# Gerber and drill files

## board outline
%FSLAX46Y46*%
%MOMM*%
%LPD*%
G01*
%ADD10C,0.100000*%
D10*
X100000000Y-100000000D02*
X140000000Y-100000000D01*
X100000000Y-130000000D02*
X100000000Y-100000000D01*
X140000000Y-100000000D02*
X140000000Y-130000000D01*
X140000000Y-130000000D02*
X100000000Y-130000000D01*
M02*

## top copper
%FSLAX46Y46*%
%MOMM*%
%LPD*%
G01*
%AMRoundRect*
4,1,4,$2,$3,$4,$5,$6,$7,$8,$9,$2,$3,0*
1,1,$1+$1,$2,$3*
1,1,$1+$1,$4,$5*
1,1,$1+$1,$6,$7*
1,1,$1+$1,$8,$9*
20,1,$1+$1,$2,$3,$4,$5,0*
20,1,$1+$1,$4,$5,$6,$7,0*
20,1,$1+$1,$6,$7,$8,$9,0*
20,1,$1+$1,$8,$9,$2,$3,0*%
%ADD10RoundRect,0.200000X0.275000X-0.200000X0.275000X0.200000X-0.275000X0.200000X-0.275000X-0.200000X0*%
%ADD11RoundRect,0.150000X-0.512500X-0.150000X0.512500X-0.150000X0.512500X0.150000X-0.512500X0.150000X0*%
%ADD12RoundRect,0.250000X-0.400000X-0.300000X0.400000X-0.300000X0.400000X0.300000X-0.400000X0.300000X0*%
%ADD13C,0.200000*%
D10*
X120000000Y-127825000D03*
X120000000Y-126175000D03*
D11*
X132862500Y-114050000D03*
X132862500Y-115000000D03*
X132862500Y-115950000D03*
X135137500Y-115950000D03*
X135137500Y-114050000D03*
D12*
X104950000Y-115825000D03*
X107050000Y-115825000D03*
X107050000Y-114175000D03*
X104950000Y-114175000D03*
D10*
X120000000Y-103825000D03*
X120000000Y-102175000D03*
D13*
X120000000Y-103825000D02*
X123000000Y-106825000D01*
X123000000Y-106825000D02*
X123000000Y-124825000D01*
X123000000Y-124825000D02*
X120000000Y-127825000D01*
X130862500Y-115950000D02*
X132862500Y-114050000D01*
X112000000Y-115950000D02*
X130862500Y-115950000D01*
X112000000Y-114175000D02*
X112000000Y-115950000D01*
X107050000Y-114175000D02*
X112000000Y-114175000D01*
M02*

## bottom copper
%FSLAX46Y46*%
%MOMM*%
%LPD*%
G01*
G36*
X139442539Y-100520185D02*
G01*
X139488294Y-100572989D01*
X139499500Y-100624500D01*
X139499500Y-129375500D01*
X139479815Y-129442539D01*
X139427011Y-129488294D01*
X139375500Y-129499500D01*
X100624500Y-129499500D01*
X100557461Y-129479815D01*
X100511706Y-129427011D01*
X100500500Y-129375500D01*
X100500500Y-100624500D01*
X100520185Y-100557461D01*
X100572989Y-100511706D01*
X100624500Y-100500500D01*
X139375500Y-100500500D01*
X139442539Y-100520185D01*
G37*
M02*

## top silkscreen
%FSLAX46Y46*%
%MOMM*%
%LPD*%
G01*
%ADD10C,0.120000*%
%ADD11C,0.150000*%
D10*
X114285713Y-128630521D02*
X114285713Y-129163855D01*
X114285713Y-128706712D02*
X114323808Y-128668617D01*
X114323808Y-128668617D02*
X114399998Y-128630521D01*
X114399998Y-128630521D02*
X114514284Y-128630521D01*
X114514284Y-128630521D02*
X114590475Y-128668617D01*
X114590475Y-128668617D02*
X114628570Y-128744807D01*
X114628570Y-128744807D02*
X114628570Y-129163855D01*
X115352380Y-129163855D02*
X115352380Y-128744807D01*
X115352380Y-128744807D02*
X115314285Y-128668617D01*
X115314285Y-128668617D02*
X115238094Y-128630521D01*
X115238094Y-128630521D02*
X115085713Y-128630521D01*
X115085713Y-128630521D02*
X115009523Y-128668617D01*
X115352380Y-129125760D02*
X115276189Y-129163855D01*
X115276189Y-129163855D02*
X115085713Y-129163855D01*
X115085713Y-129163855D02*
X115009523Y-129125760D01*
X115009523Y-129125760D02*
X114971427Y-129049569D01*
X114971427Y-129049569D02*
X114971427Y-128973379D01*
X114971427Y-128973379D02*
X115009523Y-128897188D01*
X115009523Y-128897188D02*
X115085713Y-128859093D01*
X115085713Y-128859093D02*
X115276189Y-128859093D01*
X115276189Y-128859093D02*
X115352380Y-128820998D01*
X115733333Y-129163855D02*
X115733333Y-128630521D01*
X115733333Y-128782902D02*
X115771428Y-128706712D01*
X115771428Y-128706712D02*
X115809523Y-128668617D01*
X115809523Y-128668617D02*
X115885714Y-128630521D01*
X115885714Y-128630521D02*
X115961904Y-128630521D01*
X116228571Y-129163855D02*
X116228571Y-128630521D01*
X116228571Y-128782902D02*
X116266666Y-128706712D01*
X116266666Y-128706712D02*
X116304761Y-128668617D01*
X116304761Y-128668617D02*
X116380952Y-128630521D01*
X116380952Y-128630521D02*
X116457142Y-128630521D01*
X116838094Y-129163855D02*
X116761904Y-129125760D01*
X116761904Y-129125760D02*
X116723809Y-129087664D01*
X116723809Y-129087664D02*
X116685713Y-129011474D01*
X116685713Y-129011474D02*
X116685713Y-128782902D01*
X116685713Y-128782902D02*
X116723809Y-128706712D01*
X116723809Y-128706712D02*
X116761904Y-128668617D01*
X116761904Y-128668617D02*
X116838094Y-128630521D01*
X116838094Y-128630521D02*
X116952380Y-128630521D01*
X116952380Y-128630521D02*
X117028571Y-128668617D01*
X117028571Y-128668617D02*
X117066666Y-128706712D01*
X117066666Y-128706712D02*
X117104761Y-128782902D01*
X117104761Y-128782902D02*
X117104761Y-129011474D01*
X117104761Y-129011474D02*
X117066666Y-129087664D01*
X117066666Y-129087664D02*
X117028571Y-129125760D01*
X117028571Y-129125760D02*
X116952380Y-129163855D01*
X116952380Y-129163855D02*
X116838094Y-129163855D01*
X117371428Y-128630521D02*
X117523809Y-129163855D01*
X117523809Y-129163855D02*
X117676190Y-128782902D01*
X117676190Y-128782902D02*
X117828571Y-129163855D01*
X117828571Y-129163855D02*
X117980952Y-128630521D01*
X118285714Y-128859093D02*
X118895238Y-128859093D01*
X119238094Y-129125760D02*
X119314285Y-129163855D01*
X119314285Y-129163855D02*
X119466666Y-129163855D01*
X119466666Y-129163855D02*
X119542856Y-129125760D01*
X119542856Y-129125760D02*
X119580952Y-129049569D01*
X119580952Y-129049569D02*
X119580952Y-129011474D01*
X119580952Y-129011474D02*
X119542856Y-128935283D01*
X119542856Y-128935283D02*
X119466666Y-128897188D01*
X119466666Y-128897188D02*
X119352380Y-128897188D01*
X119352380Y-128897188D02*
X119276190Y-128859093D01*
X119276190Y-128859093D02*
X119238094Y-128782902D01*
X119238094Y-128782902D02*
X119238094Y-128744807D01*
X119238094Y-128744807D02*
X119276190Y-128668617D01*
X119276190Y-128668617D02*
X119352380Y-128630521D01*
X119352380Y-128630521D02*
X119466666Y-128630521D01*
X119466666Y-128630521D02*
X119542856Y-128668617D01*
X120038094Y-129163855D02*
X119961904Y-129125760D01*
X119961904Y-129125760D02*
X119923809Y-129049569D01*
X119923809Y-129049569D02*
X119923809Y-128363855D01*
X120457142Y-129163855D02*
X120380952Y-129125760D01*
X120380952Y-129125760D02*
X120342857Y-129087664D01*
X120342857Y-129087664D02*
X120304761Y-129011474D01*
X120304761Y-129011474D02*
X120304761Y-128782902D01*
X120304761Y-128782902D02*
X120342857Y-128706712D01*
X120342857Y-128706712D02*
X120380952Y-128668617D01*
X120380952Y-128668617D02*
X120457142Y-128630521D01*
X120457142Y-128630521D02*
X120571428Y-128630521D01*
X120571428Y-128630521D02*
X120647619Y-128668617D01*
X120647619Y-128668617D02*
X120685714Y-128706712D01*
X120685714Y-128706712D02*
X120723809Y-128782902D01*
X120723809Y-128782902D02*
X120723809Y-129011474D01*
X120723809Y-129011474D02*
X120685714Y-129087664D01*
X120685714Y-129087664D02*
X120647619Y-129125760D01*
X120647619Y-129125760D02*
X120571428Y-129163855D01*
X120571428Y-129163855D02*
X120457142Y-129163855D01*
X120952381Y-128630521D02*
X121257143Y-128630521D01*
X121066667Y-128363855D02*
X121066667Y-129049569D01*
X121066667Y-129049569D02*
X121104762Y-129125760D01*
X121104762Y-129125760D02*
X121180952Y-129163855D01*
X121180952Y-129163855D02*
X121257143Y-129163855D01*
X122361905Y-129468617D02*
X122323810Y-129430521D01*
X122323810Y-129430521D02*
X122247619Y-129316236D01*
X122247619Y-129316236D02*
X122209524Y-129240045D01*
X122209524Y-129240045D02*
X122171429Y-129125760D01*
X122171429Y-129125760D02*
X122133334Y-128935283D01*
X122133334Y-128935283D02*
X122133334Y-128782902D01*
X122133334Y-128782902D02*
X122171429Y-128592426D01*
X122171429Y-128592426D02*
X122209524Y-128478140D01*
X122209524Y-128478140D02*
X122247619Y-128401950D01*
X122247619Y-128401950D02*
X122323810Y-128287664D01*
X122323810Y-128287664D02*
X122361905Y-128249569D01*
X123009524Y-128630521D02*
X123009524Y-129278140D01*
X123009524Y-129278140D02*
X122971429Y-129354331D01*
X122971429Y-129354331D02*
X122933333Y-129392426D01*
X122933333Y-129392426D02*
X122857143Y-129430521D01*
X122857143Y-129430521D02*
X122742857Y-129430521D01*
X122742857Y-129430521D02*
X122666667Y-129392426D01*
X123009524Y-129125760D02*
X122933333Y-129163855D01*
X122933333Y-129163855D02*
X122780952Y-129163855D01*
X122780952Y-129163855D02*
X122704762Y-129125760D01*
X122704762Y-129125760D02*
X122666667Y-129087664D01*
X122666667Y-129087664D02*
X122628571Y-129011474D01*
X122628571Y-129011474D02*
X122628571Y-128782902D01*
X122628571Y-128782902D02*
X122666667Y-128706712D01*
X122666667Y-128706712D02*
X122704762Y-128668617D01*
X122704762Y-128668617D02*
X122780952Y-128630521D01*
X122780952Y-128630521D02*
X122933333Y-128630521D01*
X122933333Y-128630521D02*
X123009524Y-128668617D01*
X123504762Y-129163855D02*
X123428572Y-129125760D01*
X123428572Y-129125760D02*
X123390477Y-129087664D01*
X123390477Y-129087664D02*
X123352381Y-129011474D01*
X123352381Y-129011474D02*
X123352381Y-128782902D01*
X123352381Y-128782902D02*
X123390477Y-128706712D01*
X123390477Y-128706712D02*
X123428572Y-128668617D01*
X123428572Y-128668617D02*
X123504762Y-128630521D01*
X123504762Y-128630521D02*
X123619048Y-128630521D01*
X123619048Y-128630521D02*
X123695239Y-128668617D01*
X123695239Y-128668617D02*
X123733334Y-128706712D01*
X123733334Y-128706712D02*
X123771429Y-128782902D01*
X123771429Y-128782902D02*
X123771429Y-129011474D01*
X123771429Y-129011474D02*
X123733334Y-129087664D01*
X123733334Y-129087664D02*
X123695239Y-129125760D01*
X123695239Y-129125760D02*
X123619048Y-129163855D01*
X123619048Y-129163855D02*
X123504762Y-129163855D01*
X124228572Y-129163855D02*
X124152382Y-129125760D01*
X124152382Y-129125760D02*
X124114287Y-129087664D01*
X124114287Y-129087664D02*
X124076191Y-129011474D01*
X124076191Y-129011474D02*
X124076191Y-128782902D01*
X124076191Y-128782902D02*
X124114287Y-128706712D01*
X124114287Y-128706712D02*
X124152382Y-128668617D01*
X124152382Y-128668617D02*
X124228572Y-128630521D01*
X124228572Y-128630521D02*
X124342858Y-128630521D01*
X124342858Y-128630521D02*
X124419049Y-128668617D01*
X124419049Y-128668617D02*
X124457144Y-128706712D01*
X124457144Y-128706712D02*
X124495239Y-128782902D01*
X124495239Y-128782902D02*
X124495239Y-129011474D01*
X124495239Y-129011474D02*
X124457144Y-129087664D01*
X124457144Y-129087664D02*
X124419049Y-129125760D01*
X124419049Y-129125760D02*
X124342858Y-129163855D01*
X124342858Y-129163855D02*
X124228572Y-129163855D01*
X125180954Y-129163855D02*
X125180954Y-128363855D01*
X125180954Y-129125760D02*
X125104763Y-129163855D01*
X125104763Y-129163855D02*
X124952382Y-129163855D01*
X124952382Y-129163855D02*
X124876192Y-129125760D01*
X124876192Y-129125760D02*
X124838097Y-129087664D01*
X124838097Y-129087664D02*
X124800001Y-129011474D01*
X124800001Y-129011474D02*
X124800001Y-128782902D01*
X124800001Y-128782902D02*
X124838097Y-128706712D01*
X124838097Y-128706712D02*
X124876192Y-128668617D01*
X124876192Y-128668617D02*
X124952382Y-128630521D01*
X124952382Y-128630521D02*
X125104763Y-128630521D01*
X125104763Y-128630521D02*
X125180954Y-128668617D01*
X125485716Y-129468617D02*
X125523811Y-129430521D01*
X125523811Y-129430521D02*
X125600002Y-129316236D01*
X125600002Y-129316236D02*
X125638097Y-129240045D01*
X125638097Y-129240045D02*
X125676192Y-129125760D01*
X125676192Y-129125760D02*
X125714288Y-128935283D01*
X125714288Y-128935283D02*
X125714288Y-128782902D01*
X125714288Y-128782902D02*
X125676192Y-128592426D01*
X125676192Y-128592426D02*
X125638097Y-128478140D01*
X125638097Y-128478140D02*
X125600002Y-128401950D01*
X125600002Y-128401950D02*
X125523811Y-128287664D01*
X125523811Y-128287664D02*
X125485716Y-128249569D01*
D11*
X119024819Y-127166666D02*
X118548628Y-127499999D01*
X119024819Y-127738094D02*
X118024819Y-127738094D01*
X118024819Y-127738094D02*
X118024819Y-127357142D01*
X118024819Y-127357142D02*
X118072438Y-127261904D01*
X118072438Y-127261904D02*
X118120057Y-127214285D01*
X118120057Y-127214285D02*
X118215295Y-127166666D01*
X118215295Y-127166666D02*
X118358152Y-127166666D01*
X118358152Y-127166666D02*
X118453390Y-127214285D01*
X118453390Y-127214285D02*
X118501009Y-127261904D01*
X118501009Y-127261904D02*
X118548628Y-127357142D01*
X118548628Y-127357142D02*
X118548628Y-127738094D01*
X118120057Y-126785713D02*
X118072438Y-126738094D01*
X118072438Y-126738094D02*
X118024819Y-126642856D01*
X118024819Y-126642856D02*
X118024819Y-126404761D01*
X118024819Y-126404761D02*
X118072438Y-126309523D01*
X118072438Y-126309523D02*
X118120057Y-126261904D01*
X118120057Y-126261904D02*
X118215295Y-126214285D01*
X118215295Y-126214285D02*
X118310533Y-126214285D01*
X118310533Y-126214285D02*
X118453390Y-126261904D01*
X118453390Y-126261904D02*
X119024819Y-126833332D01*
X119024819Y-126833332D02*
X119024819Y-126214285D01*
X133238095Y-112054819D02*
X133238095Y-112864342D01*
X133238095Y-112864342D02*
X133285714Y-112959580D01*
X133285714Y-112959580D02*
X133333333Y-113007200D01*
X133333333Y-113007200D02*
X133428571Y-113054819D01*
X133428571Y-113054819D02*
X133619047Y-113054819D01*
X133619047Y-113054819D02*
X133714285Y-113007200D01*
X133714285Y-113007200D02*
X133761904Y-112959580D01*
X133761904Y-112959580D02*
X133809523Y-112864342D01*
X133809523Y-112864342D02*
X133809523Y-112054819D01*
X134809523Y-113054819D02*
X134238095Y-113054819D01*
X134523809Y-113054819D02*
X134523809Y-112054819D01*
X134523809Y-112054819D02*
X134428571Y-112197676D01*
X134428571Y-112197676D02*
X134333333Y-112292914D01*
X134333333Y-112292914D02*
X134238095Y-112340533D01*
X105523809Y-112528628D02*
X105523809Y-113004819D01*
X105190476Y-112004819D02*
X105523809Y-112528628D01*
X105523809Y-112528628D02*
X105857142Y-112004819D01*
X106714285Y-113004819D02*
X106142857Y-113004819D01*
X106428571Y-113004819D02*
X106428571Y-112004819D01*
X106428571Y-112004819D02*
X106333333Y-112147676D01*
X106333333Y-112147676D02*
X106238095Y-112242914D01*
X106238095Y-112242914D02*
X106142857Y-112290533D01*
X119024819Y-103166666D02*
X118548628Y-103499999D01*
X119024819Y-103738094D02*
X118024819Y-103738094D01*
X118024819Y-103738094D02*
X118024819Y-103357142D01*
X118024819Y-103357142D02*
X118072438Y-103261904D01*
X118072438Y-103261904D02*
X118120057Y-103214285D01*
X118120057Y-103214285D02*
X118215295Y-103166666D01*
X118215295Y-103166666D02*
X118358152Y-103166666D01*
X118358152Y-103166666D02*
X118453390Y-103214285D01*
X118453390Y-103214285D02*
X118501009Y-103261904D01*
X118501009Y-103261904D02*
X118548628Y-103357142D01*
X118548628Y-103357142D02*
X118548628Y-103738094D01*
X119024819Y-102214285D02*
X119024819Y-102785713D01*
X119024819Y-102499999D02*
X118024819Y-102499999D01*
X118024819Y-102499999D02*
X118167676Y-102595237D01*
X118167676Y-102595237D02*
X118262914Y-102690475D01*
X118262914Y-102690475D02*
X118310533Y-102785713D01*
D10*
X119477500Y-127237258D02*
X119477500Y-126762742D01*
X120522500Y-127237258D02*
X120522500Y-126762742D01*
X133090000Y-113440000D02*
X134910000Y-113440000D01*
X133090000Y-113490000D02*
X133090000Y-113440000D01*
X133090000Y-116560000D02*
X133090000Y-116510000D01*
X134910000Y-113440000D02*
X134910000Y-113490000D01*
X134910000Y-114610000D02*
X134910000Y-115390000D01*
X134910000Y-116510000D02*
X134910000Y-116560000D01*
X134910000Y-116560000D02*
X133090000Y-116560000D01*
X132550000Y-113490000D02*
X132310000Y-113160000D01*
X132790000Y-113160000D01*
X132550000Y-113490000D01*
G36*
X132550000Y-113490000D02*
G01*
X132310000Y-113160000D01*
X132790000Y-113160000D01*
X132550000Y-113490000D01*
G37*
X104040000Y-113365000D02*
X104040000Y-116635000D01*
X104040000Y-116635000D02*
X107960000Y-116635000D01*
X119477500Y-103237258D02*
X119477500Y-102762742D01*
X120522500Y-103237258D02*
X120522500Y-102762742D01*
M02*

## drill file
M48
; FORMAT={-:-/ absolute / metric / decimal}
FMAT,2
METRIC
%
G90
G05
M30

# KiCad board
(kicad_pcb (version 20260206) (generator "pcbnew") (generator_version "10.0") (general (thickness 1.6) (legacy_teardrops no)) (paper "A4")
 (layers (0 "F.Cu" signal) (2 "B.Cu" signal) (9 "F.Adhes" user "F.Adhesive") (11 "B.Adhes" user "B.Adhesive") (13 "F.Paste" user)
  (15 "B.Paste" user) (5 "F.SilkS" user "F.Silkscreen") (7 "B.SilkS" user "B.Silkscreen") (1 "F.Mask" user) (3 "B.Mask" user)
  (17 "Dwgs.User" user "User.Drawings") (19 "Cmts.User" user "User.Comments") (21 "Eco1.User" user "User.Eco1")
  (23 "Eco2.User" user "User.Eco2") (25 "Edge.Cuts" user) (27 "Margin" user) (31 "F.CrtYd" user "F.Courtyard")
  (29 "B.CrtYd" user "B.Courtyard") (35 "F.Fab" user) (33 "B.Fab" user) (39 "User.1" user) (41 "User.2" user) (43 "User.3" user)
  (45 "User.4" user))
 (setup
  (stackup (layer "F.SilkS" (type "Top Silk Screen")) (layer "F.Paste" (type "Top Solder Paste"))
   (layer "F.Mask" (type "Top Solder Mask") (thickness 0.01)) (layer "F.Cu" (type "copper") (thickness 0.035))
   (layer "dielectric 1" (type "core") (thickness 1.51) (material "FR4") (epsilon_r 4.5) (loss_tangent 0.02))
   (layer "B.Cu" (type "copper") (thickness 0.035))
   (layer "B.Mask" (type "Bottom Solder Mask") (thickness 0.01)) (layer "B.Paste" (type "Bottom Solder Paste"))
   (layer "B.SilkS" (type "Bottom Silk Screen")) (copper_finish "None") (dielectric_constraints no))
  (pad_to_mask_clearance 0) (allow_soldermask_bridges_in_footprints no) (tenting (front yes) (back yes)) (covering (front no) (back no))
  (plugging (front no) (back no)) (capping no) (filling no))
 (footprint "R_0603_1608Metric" (layer "F.Cu") (at 120 127 90)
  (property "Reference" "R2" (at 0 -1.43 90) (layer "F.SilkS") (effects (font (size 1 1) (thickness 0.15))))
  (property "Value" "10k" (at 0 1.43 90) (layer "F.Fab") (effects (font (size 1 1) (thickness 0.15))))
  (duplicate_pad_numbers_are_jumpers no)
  (fp_line (start -0.237258 -0.5225) (end 0.237258 -0.5225) (stroke (width 0.12) (type solid)) (layer "F.SilkS"))
  (fp_line (start -0.237258 0.5225) (end 0.237258 0.5225) (stroke (width 0.12) (type solid)) (layer "F.SilkS"))
  (pad "1" smd roundrect (at -0.825 0 90) (size 0.8 0.95) (layers "F.Cu" "F.Mask" "F.Paste") (roundrect_rratio 0.25) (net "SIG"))
  (pad "2" smd roundrect (at 0.825 0 90) (size 0.8 0.95) (layers "F.Cu" "F.Mask" "F.Paste") (roundrect_rratio 0.25) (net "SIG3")))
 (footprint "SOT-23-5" (layer "F.Cu") (at 134 115)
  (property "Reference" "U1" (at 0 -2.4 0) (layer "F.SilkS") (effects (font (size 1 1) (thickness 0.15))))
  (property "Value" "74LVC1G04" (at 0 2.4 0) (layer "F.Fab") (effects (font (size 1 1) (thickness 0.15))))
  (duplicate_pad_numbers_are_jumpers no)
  (fp_line (start -0.91 -1.56) (end 0.91 -1.56) (stroke (width 0.12) (type solid)) (layer "F.SilkS"))
  (fp_line (start -0.91 -1.51) (end -0.91 -1.56) (stroke (width 0.12) (type solid)) (layer "F.SilkS"))
  (fp_line (start -0.91 1.56) (end -0.91 1.51) (stroke (width 0.12) (type solid)) (layer "F.SilkS"))
  (fp_line (start 0.91 -1.56) (end 0.91 -1.51) (stroke (width 0.12) (type solid)) (layer "F.SilkS"))
  (fp_line (start 0.91 -0.39) (end 0.91 0.39) (stroke (width 0.12) (type solid)) (layer "F.SilkS"))
  (fp_line (start 0.91 1.51) (end 0.91 1.56) (stroke (width 0.12) (type solid)) (layer "F.SilkS"))
  (fp_line (start 0.91 1.56) (end -0.91 1.56) (stroke (width 0.12) (type solid)) (layer "F.SilkS"))
  (fp_poly (pts (xy -1.45 -1.51) (xy -1.69 -1.84) (xy -1.21 -1.84)) (stroke (width 0.12) (type solid)) (fill yes) (layer "F.SilkS"))
  (pad "1" smd roundrect (at -1.1375 -0.95) (size 1.325 0.6) (layers "F.Cu" "F.Mask" "F.Paste") (roundrect_rratio 0.25) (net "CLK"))
  (pad "2" smd roundrect (at -1.1375 0) (size 1.325 0.6) (layers "F.Cu" "F.Mask" "F.Paste") (roundrect_rratio 0.25) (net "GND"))
  (pad "3" smd roundrect (at -1.1375 0.95) (size 1.325 0.6) (layers "F.Cu" "F.Mask" "F.Paste") (roundrect_rratio 0.25))
  (pad "4" smd roundrect (at 1.1375 0.95) (size 1.325 0.6) (layers "F.Cu" "F.Mask" "F.Paste") (roundrect_rratio 0.25))
  (pad "5" smd roundrect (at 1.1375 -0.95) (size 1.325 0.6) (layers "F.Cu" "F.Mask" "F.Paste") (roundrect_rratio 0.25) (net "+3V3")))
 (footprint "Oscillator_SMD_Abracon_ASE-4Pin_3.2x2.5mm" (layer "F.Cu") (at 106 115)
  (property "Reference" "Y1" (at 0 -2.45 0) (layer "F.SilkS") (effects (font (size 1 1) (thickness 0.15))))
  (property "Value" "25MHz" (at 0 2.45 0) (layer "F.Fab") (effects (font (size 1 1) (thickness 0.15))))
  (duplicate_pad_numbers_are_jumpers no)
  (fp_line (start -1.96 -1.635) (end -1.96 1.635) (stroke (width 0.12) (type solid)) (layer "F.SilkS"))
  (fp_line (start -1.96 1.635) (end 1.96 1.635) (stroke (width 0.12) (type solid)) (layer "F.SilkS"))
  (pad "1" smd roundrect (at -1.05 0.825) (size 1.3 1.1) (layers "F.Cu" "F.Mask" "F.Paste") (roundrect_rratio 0.227273) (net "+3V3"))
  (pad "2" smd roundrect (at 1.05 0.825) (size 1.3 1.1) (layers "F.Cu" "F.Mask" "F.Paste") (roundrect_rratio 0.227273) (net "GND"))
  (pad "3" smd roundrect (at 1.05 -0.825) (size 1.3 1.1) (layers "F.Cu" "F.Mask" "F.Paste") (roundrect_rratio 0.227273) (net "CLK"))
  (pad "4" smd roundrect (at -1.05 -0.825) (size 1.3 1.1) (layers "F.Cu" "F.Mask" "F.Paste") (roundrect_rratio 0.227273) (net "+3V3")))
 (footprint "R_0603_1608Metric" (layer "F.Cu") (at 120 103 90)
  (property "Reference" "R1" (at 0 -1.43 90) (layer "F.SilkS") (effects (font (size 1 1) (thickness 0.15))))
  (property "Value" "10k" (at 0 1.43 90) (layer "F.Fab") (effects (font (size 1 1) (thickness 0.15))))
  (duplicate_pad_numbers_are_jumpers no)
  (fp_line (start -0.237258 -0.5225) (end 0.237258 -0.5225) (stroke (width 0.12) (type solid)) (layer "F.SilkS"))
  (fp_line (start -0.237258 0.5225) (end 0.237258 0.5225) (stroke (width 0.12) (type solid)) (layer "F.SilkS"))
  (pad "1" smd roundrect (at -0.825 0 90) (size 0.8 0.95) (layers "F.Cu" "F.Mask" "F.Paste") (roundrect_rratio 0.25) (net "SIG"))
  (pad "2" smd roundrect (at 0.825 0 90) (size 0.8 0.95) (layers "F.Cu" "F.Mask" "F.Paste") (roundrect_rratio 0.25) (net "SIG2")))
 (gr_line (start 100 100) (end 140 100) (stroke (width 0.1) (type default)) (layer "Edge.Cuts"))
 (gr_line (start 100 130) (end 100 100) (stroke (width 0.1) (type default)) (layer "Edge.Cuts"))
 (gr_line (start 140 100) (end 140 130) (stroke (width 0.1) (type default)) (layer "Edge.Cuts"))
 (gr_line (start 140 130) (end 100 130) (stroke (width 0.1) (type default)) (layer "Edge.Cuts"))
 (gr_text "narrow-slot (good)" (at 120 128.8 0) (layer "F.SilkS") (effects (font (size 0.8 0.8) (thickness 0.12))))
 (segment (start 120 103.825) (end 123 106.825) (width 0.2) (layer "F.Cu") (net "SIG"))
 (segment (start 123 106.825) (end 123 124.825) (width 0.2) (layer "F.Cu") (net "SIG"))
 (segment (start 123 124.825) (end 120 127.825) (width 0.2) (layer "F.Cu") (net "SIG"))
 (segment (start 130.8625 115.95) (end 132.8625 114.05) (width 0.2) (layer "F.Cu") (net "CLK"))
 (segment (start 112 115.95) (end 130.8625 115.95) (width 0.2) (layer "F.Cu") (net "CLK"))
 (segment (start 112 114.175) (end 112 115.95) (width 0.2) (layer "F.Cu") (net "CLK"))
 (segment (start 107.05 114.175) (end 112 114.175) (width 0.2) (layer "F.Cu") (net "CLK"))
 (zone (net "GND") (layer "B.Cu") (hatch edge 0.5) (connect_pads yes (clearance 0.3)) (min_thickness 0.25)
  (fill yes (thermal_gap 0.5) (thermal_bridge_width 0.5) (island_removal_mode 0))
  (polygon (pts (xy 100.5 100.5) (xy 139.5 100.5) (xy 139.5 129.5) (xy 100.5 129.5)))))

